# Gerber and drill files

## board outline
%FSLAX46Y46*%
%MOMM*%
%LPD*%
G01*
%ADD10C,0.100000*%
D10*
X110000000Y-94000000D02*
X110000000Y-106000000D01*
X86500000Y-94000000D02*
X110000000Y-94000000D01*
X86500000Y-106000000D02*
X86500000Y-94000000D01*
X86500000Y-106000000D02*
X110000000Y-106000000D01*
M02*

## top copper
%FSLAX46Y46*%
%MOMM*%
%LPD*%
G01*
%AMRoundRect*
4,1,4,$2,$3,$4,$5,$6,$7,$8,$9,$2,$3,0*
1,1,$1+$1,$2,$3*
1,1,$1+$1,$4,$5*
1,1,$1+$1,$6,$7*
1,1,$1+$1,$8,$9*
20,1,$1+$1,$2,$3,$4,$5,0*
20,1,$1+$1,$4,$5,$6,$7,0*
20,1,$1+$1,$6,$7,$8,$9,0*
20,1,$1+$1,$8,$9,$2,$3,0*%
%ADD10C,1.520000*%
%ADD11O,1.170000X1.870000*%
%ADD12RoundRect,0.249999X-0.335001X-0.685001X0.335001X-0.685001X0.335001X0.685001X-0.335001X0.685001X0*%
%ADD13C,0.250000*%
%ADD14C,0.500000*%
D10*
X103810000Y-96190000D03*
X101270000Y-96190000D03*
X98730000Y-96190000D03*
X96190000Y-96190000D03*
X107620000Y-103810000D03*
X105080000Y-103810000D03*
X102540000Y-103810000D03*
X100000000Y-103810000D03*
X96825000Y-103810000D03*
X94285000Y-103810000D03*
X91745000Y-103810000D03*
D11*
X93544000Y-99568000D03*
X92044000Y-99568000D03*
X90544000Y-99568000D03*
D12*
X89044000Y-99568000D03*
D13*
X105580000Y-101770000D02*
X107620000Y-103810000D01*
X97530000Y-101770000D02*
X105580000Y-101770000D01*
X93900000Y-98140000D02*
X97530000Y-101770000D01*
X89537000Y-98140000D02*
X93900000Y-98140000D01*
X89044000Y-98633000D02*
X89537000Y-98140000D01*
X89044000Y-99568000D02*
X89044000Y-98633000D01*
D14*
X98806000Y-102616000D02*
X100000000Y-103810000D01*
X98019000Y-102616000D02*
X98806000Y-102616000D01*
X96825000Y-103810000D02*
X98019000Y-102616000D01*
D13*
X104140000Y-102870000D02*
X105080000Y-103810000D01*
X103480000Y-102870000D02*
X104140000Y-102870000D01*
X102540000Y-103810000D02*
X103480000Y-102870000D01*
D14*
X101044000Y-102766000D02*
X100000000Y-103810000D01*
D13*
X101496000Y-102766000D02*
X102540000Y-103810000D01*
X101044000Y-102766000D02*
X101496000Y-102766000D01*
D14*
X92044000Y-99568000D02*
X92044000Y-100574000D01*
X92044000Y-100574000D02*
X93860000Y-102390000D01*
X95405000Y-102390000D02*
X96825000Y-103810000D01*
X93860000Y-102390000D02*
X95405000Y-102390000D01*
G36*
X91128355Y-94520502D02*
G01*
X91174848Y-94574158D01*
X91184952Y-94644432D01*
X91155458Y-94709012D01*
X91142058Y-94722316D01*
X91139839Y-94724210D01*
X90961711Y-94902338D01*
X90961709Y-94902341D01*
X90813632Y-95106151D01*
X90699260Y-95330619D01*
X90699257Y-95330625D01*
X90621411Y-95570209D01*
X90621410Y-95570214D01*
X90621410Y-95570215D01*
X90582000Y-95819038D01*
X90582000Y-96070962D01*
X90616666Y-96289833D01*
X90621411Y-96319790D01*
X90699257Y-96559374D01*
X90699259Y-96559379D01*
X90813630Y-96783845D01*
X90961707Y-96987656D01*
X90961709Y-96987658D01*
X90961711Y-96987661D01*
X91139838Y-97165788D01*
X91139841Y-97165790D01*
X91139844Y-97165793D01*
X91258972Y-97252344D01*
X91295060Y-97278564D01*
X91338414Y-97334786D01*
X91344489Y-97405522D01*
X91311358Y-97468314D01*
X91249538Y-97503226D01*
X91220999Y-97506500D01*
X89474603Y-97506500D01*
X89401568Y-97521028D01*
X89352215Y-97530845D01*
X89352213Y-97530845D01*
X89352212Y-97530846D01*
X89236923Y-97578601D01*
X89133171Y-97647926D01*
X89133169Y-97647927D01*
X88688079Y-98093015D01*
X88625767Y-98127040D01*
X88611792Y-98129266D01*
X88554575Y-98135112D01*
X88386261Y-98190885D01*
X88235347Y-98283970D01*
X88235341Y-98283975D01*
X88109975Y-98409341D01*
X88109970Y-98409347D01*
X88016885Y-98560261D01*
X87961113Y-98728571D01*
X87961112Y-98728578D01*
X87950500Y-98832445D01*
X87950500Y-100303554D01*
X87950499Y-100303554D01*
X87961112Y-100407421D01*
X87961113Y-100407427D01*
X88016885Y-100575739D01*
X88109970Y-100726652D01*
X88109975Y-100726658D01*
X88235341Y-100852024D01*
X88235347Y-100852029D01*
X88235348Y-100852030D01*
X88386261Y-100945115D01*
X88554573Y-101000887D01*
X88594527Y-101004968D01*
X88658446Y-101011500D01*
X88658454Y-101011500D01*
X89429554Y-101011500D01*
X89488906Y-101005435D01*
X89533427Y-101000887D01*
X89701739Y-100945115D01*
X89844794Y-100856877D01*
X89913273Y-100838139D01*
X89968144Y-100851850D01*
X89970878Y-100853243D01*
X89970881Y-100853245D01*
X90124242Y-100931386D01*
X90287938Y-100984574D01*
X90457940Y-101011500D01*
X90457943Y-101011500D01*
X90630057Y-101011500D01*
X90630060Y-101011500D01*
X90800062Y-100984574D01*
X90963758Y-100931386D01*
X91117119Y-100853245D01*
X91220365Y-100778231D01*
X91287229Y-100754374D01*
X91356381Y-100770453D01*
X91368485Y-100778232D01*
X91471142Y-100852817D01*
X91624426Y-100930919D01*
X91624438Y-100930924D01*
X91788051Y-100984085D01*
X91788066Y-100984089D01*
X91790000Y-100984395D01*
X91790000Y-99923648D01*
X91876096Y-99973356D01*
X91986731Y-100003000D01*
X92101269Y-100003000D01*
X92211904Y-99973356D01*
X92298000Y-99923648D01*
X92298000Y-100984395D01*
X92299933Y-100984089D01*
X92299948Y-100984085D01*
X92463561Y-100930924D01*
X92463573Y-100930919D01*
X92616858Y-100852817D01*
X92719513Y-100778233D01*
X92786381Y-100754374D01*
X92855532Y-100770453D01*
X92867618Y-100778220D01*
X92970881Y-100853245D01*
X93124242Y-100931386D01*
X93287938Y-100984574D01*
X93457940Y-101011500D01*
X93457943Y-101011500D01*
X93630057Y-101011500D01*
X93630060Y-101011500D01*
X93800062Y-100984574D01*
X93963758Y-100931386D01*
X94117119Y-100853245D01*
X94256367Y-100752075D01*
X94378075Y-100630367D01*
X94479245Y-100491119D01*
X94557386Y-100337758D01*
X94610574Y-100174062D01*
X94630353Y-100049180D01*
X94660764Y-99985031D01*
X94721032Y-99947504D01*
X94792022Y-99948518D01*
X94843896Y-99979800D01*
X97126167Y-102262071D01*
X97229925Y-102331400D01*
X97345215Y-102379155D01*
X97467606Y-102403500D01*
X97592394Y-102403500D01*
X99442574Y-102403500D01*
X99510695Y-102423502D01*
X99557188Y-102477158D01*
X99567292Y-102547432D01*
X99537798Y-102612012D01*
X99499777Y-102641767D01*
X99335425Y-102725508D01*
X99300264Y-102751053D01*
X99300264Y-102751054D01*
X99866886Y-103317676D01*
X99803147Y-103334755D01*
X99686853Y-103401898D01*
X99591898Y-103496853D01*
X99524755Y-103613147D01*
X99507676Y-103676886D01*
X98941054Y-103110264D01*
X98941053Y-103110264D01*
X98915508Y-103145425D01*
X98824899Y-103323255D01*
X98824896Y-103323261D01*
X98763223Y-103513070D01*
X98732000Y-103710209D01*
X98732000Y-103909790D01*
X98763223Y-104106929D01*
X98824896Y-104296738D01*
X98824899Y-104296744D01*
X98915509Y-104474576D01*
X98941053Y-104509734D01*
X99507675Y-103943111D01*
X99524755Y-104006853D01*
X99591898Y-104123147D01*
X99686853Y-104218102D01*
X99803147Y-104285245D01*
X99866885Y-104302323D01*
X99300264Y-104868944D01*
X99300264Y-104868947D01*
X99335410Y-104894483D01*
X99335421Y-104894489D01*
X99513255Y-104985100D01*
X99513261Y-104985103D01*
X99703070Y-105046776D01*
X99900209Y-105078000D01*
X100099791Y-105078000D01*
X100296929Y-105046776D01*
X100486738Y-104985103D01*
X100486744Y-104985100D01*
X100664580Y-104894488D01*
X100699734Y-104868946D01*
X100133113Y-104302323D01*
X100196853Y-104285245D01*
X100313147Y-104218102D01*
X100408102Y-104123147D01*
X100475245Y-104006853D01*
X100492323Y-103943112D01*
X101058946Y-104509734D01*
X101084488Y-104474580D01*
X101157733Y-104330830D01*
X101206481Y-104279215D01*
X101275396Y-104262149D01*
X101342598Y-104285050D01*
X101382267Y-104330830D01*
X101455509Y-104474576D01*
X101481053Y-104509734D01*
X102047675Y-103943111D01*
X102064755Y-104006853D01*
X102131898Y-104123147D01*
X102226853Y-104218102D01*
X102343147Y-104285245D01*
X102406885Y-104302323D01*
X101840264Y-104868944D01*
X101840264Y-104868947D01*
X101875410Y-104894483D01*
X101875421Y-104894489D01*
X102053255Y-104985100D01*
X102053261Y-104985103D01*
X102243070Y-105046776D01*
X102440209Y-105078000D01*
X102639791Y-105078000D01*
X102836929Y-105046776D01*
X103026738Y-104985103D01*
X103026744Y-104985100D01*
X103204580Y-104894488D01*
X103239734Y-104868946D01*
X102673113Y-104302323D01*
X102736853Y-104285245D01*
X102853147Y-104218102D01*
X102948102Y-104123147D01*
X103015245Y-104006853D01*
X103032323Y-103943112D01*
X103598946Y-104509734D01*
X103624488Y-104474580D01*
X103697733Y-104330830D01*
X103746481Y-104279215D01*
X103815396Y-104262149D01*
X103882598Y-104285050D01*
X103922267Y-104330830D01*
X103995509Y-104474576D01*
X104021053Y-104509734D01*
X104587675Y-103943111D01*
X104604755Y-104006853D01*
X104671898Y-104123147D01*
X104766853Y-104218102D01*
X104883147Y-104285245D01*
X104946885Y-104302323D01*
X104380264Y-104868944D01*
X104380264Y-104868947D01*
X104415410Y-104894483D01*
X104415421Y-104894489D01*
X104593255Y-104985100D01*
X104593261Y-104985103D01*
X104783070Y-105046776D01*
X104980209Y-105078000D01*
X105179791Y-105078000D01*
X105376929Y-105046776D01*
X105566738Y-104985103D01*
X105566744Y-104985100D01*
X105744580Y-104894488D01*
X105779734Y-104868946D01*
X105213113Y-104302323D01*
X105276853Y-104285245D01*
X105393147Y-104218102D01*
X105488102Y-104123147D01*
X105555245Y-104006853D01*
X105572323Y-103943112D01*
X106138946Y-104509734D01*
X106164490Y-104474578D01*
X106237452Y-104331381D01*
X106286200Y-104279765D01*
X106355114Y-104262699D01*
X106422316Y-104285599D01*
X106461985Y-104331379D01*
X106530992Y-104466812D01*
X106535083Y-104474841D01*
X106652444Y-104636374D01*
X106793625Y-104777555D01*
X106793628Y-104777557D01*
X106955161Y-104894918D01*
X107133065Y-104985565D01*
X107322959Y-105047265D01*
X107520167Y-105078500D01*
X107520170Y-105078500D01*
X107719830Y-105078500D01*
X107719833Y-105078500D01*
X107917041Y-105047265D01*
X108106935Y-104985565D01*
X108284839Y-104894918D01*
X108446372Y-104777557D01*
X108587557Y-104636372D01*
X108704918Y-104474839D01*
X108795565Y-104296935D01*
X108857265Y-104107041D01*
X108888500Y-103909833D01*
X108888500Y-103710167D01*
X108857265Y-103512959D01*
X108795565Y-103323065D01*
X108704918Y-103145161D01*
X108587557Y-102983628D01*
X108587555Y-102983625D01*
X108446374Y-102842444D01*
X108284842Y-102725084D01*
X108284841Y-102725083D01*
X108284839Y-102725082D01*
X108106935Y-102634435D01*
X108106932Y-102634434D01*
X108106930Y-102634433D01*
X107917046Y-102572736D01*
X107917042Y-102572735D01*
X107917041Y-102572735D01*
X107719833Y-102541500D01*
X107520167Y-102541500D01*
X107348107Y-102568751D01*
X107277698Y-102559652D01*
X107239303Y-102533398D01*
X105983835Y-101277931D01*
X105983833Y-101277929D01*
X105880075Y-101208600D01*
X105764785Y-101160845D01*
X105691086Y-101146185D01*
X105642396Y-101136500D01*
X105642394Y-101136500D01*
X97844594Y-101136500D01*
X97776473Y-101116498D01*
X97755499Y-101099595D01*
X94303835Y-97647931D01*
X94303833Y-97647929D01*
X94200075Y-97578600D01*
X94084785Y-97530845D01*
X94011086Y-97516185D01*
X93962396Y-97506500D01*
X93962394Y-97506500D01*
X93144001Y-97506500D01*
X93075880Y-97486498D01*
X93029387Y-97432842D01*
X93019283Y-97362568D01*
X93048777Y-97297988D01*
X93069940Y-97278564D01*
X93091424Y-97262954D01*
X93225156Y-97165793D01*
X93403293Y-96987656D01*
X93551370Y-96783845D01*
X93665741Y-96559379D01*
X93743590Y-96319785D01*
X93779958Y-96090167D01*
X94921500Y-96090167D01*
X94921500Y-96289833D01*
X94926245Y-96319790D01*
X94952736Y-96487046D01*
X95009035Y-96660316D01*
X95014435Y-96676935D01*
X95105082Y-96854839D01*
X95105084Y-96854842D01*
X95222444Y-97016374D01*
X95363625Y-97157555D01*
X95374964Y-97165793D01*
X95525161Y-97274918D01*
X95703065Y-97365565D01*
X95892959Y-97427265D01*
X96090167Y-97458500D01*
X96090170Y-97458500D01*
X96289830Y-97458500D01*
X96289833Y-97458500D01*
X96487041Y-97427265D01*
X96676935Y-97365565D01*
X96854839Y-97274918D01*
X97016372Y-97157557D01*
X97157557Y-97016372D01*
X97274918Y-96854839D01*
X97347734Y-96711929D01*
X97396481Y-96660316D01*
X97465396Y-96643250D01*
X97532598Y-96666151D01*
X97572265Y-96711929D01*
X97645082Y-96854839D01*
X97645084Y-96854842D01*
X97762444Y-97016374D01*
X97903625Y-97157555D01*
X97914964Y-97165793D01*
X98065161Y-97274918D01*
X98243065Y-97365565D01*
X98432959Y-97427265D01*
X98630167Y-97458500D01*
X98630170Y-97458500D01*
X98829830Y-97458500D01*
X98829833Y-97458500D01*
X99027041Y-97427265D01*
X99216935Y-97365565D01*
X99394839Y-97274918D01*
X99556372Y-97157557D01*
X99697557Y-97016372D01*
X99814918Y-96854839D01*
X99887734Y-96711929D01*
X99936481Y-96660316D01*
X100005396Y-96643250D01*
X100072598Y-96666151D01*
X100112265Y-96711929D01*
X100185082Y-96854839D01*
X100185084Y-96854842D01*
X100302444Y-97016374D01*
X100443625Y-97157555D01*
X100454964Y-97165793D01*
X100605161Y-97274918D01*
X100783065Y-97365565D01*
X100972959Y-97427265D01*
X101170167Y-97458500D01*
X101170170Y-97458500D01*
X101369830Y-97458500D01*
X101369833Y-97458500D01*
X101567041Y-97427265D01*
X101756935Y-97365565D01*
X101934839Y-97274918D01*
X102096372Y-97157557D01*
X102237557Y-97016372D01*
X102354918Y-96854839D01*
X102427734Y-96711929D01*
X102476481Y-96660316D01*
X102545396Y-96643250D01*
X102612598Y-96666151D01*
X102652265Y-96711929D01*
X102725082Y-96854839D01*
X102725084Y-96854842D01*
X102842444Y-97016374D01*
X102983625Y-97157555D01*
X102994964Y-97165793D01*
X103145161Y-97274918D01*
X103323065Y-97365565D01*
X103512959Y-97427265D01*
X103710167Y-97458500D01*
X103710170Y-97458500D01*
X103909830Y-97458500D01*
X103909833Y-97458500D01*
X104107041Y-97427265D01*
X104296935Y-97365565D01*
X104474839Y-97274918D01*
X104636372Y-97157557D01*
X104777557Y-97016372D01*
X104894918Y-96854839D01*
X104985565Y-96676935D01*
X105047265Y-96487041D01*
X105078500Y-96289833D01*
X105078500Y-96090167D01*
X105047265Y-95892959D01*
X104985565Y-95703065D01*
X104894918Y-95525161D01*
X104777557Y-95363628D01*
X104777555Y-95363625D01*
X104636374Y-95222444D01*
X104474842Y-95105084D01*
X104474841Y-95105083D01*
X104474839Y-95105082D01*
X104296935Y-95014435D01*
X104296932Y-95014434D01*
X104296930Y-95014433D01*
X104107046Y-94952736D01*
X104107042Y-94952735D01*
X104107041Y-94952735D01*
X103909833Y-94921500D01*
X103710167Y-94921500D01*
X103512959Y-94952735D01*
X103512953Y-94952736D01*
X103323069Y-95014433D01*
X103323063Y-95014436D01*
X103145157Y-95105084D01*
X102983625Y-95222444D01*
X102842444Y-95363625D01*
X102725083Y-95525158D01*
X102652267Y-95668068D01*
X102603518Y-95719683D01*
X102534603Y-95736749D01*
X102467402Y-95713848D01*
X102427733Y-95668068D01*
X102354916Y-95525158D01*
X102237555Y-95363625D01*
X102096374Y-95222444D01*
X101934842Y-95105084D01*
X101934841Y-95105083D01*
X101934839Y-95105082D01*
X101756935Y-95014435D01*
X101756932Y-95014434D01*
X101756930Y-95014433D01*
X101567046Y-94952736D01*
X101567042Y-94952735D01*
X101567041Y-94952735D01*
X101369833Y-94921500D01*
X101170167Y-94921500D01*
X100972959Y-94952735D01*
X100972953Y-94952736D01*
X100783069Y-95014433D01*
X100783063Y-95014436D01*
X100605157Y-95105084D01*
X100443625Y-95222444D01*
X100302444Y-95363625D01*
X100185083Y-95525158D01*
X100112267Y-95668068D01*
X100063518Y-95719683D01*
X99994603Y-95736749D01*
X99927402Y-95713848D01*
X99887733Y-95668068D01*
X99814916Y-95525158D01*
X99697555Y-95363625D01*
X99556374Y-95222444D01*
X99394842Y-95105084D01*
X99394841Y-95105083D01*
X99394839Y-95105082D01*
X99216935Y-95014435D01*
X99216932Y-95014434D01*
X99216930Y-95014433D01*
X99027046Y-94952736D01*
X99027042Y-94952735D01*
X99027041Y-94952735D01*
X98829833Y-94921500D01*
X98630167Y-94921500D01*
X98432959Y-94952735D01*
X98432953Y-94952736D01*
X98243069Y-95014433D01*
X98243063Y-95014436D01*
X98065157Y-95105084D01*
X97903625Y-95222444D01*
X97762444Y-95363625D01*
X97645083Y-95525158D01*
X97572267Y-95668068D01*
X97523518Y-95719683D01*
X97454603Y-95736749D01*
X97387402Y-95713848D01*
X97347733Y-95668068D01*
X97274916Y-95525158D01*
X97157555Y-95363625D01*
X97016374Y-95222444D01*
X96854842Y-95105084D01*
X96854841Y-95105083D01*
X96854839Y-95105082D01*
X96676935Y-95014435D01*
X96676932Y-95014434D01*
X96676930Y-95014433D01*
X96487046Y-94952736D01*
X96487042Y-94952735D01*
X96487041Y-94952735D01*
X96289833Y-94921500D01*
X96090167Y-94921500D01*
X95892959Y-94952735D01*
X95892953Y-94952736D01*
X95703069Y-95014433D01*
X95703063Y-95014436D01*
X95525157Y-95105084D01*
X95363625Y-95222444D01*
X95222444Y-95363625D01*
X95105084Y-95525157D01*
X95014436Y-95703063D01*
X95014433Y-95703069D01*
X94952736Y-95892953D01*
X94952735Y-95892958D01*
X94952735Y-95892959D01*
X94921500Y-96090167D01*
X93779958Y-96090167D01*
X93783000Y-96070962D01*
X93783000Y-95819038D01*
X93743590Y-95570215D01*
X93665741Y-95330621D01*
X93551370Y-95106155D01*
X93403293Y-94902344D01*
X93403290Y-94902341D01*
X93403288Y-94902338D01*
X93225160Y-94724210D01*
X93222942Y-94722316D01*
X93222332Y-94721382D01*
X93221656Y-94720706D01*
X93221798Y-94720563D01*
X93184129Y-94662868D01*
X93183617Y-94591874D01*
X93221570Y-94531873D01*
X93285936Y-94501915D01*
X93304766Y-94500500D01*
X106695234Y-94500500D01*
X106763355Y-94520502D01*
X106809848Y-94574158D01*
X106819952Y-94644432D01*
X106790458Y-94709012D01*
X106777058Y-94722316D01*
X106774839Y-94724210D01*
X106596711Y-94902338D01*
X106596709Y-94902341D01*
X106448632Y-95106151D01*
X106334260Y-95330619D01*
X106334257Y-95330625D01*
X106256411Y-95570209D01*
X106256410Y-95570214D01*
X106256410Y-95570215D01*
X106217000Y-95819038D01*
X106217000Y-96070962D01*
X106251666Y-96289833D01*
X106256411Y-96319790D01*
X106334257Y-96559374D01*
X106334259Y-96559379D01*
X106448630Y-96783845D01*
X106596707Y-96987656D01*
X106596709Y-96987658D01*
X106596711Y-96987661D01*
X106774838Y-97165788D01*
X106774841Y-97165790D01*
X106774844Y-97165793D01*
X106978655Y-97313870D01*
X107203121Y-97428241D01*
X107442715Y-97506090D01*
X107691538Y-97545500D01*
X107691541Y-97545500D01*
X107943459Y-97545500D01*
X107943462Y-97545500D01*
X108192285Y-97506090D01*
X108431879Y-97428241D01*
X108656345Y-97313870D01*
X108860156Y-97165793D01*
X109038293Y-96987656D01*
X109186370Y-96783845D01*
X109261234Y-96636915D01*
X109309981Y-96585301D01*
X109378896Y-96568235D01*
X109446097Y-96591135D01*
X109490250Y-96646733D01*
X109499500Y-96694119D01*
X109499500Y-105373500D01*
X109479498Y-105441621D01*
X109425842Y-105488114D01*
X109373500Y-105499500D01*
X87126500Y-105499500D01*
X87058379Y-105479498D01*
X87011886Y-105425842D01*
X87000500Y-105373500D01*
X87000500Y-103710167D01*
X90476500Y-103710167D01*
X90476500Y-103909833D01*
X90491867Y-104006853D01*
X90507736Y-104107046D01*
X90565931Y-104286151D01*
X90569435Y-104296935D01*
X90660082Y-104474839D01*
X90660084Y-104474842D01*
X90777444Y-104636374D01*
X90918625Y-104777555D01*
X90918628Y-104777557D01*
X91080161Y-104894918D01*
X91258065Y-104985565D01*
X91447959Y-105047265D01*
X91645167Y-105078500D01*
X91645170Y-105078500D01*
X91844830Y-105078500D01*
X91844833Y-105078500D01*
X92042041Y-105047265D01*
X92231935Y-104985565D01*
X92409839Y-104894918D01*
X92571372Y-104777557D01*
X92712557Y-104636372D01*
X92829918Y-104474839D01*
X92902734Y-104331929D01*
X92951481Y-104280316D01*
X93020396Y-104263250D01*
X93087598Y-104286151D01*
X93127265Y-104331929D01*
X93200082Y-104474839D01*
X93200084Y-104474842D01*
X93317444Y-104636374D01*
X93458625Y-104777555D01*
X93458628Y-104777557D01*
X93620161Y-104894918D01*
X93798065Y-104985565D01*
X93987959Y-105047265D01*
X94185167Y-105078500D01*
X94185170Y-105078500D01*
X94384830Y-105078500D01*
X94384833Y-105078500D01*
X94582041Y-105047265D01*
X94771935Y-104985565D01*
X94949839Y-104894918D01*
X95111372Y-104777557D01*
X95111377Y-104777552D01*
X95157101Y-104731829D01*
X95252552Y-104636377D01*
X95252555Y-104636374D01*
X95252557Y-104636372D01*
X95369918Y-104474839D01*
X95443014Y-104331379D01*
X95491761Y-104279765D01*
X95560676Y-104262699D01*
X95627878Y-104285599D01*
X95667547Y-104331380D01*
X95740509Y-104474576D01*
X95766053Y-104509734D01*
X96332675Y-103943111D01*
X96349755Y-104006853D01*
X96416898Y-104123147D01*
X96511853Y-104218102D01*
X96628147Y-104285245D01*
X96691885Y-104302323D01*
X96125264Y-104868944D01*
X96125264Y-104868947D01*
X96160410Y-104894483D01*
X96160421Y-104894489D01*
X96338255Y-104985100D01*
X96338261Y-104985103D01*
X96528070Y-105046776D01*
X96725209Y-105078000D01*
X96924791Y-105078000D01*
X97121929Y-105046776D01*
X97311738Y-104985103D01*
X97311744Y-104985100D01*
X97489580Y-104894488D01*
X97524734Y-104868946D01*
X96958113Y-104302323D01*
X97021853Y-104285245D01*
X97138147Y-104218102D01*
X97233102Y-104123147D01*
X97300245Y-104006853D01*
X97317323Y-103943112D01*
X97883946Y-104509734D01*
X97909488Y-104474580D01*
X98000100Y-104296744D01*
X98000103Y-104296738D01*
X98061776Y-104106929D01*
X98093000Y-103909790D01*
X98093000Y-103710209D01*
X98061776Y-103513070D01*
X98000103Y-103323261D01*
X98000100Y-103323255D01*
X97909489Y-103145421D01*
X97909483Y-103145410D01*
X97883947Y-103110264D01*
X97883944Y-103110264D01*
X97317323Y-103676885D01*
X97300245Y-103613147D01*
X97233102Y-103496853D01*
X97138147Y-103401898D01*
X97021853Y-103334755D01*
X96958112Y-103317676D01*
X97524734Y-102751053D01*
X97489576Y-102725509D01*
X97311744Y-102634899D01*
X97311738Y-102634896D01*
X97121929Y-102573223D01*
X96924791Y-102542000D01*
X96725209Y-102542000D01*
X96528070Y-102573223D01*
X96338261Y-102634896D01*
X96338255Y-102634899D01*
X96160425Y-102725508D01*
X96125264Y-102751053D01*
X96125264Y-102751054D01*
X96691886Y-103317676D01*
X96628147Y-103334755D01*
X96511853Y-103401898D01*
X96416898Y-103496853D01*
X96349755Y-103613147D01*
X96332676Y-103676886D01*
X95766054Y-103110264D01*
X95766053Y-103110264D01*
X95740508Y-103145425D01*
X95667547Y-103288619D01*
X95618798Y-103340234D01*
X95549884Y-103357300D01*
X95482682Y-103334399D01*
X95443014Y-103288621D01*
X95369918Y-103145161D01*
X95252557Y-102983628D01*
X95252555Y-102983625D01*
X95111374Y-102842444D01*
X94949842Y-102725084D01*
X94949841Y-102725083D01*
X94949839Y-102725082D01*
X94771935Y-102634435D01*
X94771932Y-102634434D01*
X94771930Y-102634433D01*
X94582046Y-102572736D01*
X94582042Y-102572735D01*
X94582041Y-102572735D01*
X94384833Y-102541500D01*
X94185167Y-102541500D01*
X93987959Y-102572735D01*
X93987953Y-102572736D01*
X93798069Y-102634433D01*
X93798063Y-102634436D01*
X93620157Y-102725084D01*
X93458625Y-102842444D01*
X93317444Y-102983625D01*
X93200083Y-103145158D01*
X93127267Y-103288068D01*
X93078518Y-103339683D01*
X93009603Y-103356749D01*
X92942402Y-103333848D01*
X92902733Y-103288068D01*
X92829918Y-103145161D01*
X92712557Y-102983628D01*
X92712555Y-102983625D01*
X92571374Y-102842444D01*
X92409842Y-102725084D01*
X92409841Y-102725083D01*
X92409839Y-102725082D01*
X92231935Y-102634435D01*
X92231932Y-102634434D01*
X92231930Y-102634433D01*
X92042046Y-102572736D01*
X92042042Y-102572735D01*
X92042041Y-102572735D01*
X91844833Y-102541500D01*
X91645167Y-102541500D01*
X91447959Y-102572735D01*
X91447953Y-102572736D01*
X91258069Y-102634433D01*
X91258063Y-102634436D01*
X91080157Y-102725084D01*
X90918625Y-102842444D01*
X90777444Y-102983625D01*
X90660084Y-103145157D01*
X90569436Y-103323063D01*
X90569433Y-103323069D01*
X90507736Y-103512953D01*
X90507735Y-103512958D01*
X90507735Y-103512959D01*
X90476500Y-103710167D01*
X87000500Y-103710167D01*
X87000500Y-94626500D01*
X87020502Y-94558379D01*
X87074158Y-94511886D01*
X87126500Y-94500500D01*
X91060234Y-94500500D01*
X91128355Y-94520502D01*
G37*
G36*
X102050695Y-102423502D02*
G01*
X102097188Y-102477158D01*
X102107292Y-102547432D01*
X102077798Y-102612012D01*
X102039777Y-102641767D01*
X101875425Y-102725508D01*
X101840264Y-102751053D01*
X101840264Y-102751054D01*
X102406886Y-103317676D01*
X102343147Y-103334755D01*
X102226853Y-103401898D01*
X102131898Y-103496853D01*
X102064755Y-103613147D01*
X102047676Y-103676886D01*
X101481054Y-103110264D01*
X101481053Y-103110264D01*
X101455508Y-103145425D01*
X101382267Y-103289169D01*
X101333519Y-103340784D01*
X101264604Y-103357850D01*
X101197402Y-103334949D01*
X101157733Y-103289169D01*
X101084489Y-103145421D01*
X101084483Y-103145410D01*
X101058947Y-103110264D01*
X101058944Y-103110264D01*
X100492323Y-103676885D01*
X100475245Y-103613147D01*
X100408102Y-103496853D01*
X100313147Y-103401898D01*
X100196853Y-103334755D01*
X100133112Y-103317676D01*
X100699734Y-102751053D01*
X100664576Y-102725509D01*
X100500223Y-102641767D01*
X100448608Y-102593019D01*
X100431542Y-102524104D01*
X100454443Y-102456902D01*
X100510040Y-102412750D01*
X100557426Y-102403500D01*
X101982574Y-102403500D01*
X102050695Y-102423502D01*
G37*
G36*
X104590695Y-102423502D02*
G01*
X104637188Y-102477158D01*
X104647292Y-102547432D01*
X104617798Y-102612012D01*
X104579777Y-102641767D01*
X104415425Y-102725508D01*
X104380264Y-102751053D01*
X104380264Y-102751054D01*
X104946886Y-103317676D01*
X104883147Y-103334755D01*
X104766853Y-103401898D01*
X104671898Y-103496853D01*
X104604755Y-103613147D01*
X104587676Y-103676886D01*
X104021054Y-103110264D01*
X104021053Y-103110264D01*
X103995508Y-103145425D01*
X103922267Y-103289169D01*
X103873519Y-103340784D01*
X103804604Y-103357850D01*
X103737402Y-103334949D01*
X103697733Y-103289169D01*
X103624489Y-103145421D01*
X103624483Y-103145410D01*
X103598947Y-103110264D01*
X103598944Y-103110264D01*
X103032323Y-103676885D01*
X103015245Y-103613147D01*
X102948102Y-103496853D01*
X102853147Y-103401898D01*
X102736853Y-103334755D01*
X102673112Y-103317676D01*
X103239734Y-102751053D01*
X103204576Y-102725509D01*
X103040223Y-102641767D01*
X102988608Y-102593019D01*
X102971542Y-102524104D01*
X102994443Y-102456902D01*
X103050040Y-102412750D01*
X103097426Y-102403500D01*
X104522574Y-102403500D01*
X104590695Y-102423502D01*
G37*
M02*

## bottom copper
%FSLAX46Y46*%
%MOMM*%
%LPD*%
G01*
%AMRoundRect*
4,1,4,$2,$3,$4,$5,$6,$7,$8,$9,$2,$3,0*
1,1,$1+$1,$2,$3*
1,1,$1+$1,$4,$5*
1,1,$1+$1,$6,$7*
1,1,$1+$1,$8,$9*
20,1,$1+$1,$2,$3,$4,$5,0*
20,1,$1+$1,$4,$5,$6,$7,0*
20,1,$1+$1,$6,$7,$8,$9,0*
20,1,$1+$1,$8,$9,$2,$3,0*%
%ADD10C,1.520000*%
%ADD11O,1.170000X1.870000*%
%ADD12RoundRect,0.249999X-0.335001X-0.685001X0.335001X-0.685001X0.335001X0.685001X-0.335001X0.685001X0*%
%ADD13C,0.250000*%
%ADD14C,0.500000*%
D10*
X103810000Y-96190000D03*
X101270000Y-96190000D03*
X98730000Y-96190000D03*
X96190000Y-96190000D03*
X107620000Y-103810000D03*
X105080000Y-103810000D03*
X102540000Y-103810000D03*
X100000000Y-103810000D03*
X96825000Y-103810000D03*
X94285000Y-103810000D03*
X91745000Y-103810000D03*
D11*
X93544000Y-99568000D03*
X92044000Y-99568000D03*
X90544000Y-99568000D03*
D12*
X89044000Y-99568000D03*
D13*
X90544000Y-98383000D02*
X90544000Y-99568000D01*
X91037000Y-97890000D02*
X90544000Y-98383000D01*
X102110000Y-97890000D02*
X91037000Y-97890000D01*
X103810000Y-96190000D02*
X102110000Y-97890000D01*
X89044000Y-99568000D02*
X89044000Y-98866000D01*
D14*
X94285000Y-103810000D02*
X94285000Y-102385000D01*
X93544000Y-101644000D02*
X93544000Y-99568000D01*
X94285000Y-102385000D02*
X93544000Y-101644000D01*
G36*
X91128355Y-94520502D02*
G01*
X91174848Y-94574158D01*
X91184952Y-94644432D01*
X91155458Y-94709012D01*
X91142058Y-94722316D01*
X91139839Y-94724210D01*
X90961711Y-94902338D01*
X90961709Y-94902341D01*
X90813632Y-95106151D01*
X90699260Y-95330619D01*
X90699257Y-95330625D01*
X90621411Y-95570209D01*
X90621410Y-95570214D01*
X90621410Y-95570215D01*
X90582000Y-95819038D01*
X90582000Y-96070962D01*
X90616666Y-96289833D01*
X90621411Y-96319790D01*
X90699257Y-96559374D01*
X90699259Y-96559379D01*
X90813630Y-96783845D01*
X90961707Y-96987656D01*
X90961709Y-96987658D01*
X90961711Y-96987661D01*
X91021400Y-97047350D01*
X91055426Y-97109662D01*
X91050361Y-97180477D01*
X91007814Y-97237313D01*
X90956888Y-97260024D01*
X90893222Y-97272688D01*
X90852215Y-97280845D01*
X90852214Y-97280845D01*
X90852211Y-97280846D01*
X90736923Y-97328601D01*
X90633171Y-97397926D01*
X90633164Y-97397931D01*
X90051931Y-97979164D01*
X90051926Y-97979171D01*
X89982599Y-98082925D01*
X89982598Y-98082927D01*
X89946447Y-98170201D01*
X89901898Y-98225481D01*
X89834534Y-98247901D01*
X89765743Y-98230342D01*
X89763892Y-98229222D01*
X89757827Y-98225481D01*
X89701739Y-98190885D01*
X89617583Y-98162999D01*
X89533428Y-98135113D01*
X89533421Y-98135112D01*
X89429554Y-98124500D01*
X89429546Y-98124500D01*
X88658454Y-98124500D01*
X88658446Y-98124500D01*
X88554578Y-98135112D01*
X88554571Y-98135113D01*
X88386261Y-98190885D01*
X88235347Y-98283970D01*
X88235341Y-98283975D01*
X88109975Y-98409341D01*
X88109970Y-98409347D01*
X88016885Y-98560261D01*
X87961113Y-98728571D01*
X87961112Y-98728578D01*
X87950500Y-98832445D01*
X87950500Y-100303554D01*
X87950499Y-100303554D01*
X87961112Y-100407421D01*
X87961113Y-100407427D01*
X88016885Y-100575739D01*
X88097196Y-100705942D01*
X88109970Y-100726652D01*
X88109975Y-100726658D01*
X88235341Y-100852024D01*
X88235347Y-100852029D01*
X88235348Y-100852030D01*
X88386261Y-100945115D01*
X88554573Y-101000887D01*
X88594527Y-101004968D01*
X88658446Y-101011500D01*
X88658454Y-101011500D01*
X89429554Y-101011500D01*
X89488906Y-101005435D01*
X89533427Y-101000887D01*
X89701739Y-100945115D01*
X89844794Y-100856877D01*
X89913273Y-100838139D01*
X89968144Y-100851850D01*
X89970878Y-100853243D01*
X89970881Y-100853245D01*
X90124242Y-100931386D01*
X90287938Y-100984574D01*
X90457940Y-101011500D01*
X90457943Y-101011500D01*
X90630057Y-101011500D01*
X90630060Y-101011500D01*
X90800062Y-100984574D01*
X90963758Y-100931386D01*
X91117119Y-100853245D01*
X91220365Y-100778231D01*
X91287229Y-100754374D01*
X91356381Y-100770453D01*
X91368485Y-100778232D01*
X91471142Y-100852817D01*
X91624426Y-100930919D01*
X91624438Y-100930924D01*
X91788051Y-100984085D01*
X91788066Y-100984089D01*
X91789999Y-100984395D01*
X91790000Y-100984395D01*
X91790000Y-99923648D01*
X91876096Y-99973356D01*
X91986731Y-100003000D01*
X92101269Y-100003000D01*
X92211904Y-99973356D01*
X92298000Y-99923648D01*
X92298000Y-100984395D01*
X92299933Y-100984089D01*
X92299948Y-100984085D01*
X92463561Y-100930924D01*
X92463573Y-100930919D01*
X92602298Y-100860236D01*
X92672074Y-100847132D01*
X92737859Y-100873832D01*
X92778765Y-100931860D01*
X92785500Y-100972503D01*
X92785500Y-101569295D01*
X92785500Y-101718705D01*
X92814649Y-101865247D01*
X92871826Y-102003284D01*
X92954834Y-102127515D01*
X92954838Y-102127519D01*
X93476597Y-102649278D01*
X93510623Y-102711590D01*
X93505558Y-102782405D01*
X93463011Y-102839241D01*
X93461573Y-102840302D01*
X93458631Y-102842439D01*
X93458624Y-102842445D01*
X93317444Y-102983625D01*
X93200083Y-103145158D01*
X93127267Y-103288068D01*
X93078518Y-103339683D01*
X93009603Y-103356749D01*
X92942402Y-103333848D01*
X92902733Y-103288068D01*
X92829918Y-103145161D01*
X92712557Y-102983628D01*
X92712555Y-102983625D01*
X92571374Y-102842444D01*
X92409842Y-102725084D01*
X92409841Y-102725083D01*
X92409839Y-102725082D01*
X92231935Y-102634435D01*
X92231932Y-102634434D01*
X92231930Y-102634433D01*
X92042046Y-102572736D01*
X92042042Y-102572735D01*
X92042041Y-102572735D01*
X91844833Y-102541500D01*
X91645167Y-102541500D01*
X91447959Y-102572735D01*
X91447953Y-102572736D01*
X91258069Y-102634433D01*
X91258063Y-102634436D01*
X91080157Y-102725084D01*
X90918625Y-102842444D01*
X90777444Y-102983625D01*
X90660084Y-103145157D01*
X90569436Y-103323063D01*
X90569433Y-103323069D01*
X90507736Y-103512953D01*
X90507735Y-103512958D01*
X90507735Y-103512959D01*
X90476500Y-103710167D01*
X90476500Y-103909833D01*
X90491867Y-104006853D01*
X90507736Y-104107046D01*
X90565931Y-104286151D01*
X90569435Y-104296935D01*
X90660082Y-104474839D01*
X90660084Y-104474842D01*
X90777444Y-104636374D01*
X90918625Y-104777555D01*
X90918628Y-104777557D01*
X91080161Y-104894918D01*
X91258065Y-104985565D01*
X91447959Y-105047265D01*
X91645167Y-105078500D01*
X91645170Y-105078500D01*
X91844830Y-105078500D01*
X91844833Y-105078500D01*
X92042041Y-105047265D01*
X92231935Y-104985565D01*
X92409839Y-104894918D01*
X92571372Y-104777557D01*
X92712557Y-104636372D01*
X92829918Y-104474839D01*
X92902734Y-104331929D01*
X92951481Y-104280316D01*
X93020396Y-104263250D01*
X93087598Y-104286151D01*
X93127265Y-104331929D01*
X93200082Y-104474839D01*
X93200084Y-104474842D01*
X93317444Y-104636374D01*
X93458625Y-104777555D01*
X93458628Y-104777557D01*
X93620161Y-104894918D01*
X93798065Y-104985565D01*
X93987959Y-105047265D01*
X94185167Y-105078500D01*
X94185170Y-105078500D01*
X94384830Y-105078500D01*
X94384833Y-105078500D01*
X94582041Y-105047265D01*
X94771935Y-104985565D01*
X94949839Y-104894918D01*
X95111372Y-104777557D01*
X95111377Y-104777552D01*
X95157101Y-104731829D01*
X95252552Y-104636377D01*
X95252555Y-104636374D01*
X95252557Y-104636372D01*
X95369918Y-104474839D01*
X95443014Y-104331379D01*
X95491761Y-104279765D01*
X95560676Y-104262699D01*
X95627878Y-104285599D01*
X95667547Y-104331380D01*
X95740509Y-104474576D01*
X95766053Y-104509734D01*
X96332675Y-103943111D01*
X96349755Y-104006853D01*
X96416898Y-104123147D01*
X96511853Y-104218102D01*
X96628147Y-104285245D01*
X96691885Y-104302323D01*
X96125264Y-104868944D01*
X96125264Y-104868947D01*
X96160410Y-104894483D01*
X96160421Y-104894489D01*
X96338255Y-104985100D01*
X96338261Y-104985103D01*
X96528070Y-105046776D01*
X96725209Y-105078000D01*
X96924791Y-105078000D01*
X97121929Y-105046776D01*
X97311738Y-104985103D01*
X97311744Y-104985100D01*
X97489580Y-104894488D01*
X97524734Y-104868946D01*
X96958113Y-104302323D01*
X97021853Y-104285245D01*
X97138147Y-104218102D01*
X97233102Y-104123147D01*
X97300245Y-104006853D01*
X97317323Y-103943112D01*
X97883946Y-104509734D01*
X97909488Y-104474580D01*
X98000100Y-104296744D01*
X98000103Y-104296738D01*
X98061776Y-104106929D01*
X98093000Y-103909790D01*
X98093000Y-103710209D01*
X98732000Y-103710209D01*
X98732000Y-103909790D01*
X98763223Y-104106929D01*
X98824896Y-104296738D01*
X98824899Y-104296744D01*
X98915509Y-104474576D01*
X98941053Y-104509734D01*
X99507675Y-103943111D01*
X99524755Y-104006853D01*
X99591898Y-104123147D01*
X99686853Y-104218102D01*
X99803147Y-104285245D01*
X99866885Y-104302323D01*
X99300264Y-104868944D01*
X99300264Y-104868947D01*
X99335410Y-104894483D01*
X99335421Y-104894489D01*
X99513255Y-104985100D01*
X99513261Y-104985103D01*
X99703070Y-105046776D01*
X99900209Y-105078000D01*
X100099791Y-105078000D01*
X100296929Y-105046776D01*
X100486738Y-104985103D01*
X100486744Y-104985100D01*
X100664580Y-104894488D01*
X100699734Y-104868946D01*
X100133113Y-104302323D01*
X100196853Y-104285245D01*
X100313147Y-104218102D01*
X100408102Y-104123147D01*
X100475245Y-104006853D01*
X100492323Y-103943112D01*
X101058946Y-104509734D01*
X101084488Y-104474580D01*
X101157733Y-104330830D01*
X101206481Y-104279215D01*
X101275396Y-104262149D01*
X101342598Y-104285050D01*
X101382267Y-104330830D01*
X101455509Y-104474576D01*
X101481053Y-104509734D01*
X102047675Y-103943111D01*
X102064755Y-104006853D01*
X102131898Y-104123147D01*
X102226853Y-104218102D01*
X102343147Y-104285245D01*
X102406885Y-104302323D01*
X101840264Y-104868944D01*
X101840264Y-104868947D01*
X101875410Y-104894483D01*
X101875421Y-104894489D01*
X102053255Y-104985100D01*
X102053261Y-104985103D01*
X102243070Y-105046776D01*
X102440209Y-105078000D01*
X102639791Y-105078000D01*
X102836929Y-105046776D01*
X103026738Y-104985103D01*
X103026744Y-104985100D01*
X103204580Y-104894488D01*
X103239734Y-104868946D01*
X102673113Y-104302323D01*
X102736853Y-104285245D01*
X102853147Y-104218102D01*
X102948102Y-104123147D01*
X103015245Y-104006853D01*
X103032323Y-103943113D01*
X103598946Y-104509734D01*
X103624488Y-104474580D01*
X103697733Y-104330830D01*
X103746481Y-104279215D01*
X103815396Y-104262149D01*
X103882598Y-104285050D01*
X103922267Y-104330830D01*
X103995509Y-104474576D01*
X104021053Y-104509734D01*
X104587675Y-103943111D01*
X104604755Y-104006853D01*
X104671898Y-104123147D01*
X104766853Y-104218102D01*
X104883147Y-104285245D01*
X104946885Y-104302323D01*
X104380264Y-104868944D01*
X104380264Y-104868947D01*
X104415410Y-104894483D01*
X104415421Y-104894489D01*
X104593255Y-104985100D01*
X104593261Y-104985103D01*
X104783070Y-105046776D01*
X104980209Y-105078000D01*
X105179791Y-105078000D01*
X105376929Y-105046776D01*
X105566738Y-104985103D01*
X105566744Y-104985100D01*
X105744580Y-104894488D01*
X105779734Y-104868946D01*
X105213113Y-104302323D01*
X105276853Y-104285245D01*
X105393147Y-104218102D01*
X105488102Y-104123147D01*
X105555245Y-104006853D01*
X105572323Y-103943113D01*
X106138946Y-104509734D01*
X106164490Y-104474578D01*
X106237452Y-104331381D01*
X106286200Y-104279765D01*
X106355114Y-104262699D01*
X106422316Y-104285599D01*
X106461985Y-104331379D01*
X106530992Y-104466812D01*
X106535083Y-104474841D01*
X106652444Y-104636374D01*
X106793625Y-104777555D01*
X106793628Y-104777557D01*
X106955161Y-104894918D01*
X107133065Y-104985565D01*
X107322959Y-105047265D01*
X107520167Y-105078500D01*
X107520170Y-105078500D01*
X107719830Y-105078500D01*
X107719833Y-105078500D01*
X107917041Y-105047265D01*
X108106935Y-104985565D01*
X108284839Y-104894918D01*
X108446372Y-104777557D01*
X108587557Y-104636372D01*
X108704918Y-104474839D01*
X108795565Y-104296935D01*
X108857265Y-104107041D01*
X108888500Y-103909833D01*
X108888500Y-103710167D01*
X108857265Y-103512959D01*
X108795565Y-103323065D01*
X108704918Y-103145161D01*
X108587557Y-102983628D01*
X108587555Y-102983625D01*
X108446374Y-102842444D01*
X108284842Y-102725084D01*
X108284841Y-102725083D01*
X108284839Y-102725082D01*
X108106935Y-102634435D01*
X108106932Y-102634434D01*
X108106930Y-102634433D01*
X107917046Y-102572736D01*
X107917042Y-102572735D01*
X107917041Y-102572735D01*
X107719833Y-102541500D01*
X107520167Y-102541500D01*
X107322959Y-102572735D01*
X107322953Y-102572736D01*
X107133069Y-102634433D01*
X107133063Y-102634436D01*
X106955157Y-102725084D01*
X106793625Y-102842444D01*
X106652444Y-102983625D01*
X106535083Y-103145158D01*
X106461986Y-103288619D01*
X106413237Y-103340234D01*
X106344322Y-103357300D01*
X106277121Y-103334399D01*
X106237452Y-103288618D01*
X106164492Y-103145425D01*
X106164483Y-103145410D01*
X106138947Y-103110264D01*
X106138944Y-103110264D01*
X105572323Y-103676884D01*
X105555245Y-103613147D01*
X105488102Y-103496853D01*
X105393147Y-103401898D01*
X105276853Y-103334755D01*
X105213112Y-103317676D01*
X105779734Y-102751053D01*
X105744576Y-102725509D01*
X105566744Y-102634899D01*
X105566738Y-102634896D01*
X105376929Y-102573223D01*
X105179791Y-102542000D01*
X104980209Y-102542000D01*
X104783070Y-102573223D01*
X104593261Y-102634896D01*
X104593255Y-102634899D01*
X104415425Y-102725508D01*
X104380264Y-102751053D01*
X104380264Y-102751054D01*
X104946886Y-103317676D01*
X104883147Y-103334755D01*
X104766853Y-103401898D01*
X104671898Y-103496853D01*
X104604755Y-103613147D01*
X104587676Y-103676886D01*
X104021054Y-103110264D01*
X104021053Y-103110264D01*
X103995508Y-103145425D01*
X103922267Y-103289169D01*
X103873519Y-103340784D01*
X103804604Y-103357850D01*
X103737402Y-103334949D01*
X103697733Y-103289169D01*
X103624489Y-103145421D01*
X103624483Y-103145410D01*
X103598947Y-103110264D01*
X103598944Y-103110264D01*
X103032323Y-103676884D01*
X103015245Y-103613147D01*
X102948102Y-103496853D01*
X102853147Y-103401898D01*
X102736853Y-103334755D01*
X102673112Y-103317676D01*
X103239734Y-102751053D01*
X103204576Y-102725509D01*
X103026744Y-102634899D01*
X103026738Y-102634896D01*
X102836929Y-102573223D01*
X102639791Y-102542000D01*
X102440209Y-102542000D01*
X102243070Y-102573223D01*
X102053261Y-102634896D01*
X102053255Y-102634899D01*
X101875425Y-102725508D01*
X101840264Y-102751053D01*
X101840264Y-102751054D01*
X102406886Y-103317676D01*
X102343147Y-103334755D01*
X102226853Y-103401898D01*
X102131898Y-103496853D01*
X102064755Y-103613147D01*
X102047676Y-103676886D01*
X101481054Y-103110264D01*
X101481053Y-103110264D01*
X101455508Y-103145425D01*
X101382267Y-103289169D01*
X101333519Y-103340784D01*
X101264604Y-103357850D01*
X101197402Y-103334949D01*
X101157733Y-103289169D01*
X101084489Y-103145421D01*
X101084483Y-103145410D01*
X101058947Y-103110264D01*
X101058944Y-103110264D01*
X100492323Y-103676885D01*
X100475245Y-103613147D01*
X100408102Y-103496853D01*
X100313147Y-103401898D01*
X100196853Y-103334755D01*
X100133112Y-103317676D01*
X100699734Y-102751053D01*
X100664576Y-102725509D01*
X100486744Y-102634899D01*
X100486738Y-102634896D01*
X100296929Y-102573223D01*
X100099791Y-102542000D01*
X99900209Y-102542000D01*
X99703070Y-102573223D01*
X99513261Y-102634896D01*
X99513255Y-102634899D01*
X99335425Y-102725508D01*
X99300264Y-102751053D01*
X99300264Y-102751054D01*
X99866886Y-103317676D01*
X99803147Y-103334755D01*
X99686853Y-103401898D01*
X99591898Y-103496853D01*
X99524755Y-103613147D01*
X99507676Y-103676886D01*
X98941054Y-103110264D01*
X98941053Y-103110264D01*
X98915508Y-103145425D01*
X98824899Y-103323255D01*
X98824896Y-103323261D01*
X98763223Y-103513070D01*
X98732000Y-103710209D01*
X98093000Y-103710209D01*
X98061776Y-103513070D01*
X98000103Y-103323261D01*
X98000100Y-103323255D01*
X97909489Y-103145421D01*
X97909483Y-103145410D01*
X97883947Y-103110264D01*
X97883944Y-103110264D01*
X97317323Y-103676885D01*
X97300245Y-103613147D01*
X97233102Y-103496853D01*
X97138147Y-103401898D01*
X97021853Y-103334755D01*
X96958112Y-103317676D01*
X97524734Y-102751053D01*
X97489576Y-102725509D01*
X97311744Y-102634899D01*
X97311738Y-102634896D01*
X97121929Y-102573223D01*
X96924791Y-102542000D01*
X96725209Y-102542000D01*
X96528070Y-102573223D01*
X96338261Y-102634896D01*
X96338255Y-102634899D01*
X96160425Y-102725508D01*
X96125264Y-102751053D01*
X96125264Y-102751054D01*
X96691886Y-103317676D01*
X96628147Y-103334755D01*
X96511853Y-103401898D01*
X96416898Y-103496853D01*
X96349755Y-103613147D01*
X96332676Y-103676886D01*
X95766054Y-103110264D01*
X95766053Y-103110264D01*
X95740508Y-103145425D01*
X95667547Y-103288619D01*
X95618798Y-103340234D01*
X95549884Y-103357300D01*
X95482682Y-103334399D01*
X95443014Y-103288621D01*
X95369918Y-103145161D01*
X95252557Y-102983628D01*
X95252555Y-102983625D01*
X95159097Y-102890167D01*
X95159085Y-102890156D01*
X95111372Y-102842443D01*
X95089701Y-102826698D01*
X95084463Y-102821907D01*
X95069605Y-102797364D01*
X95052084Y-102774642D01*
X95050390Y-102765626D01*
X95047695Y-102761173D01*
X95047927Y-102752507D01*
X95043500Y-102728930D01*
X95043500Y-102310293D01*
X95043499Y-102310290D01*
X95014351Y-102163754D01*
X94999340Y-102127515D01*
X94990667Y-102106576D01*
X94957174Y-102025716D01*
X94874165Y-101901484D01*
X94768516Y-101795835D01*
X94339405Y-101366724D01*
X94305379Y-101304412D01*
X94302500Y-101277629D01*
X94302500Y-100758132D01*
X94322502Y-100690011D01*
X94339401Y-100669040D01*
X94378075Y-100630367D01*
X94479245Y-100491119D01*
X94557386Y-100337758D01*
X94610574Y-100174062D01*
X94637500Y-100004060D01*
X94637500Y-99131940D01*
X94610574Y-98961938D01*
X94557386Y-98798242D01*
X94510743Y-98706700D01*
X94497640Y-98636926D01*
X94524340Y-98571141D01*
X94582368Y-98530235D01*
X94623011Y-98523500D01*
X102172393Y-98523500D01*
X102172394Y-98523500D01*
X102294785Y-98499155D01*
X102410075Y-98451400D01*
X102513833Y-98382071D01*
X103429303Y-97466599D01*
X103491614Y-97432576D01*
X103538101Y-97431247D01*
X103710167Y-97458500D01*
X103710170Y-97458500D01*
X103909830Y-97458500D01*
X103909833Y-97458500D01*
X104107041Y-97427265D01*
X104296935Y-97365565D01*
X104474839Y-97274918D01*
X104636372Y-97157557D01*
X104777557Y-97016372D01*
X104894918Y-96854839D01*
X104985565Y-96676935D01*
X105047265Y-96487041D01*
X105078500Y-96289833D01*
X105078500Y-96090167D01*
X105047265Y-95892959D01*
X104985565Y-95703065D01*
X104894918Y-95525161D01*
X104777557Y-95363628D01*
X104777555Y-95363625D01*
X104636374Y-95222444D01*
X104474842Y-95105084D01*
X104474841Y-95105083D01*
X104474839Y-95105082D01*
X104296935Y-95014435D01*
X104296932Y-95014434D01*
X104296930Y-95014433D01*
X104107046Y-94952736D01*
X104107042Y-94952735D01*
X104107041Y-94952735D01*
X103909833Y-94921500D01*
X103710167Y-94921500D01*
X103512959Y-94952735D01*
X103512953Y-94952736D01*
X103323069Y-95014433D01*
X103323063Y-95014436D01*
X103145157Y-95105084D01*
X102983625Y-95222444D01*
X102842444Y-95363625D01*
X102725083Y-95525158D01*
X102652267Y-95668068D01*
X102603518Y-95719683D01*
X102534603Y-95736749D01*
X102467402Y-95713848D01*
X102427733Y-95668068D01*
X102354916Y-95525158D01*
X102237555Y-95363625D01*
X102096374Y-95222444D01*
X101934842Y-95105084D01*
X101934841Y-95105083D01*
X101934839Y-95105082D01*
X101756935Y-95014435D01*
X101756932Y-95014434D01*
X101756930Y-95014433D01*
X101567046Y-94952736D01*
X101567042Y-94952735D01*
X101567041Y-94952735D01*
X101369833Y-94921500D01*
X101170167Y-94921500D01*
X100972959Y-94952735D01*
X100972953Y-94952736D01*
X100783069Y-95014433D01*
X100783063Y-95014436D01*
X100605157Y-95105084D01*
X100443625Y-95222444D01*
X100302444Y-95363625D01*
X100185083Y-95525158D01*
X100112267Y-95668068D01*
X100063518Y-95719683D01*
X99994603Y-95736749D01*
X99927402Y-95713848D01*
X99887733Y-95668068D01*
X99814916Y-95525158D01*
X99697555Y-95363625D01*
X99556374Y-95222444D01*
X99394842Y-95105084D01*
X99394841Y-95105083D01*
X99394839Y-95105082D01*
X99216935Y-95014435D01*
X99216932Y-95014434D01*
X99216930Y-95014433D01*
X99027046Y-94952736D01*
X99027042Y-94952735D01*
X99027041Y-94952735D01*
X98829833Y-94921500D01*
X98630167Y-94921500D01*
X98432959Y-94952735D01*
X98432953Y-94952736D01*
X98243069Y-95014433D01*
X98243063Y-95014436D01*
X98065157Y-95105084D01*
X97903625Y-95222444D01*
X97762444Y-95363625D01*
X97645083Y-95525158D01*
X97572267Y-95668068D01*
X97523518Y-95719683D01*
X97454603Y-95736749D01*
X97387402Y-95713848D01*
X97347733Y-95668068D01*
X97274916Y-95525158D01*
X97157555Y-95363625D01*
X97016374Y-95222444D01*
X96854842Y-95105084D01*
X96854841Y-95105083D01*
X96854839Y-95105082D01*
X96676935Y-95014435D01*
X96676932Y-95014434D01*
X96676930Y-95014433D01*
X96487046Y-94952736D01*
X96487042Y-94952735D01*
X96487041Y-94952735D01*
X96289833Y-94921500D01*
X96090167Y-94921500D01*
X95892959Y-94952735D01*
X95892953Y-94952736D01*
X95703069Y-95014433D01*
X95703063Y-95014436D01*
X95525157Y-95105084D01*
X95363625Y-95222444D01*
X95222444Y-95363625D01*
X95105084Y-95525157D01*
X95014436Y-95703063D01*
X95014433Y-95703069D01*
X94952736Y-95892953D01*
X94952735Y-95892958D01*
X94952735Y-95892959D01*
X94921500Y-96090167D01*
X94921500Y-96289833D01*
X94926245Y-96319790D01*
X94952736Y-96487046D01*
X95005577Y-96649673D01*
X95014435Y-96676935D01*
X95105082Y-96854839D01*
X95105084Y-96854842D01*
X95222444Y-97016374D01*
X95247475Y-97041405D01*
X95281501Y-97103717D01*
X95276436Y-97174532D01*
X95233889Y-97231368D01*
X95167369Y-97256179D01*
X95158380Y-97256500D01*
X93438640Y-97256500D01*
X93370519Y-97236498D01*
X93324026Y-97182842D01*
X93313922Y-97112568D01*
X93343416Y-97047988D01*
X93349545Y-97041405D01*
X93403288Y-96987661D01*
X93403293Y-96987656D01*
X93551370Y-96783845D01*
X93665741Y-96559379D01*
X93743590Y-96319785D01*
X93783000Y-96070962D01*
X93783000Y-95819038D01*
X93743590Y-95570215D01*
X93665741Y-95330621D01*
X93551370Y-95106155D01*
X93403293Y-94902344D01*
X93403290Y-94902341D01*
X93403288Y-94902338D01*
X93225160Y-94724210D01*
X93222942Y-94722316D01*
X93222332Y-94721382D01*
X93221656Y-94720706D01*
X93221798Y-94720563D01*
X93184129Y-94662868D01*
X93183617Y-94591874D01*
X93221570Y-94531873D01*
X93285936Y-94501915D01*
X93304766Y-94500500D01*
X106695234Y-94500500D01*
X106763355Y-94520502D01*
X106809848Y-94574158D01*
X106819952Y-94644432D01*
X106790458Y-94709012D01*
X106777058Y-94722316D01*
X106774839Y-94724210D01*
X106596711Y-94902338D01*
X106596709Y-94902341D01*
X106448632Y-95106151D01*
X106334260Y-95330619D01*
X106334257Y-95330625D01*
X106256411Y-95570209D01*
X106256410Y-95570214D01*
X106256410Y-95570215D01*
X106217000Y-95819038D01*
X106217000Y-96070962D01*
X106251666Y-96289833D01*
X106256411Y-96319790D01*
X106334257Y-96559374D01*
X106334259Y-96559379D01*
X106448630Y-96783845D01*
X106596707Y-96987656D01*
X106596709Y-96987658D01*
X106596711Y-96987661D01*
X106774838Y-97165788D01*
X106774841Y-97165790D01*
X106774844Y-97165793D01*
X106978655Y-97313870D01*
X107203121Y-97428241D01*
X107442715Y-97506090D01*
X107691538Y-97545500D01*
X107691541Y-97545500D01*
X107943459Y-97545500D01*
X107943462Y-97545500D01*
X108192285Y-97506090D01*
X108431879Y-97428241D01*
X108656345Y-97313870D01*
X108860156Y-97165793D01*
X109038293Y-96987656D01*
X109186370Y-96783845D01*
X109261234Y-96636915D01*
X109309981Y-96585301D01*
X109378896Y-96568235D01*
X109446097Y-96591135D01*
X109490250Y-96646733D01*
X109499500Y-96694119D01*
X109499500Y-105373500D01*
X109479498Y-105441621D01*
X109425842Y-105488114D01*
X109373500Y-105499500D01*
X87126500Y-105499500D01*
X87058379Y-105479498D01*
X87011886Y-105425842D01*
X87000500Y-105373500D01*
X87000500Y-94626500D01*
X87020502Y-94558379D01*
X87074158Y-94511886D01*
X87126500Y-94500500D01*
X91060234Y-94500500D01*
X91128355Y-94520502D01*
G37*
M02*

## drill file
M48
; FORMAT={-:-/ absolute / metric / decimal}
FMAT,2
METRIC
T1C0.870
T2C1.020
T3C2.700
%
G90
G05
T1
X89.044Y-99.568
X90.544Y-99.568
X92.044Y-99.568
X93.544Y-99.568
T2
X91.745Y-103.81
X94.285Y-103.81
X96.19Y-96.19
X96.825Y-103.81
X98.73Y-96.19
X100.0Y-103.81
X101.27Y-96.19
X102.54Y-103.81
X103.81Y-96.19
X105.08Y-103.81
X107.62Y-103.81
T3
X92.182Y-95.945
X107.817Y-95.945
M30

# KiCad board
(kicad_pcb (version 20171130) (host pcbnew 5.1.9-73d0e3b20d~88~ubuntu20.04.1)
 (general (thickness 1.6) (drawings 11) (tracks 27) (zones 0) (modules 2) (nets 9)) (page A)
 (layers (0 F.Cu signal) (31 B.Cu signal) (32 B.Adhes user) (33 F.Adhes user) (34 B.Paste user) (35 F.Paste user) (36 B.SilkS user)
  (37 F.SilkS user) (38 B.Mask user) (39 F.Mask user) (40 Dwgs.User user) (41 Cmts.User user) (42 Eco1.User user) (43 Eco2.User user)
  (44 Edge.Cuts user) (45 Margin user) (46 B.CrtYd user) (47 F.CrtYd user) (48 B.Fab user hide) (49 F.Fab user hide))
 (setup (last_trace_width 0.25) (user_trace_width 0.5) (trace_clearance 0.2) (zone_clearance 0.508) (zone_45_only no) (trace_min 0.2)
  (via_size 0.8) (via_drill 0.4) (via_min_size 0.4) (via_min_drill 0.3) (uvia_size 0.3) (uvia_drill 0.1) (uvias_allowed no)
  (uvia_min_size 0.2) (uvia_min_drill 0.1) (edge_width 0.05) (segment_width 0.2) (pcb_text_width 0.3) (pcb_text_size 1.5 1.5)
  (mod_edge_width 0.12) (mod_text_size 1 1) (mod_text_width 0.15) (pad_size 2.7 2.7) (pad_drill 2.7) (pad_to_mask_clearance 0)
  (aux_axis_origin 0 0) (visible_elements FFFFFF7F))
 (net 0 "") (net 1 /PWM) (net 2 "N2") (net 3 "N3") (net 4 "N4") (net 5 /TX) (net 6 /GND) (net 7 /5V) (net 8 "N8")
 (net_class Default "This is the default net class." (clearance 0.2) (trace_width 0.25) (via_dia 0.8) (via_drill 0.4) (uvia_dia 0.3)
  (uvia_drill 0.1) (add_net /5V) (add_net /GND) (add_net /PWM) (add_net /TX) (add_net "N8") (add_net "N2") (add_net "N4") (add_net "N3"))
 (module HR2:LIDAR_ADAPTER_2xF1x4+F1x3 (layer F.Cu) (at 100 100)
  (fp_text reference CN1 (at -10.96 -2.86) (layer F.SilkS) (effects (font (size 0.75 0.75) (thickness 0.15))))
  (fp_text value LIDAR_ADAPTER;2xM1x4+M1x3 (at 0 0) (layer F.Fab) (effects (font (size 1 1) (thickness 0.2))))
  (pad "" np_thru_hole circle (at -7.8175 -4.055) (size 2.7 2.7) (drill 2.7) (layers *.Cu *.Mask))
  (pad "" np_thru_hole circle (at 7.8175 -4.055) (size 2.7 2.7) (drill 2.7) (layers *.Cu *.Mask))
  (pad 11 thru_hole circle (at 3.81 -3.81) (size 1.52 1.52) (drill 1.02) (layers *.Cu *.Mask) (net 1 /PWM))
  (pad 10 thru_hole circle (at 1.27 -3.81) (size 1.52 1.52) (drill 1.02) (layers *.Cu *.Mask) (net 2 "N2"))
  (pad 9 thru_hole circle (at -1.27 -3.81) (size 1.52 1.52) (drill 1.02) (layers *.Cu *.Mask) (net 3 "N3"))
  (pad 8 thru_hole circle (at -3.81 -3.81) (size 1.52 1.52) (drill 1.02) (layers *.Cu *.Mask) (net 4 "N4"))
  (pad 7 thru_hole circle (at 7.62 3.81) (size 1.52 1.52) (drill 1.02) (layers *.Cu *.Mask) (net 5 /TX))
  (pad 6 thru_hole circle (at 5.08 3.81) (size 1.52 1.52) (drill 1.02) (layers *.Cu *.Mask) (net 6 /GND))
  (pad 5 thru_hole circle (at 2.54 3.81) (size 1.52 1.52) (drill 1.02) (layers *.Cu *.Mask) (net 6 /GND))
  (pad 4 thru_hole circle (at 0 3.81) (size 1.52 1.52) (drill 1.02) (layers *.Cu *.Mask) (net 6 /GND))
  (pad 3 thru_hole circle (at -3.175 3.81) (size 1.52 1.52) (drill 1.02) (layers *.Cu *.Mask) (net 6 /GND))
  (pad 2 thru_hole circle (at -5.715 3.81) (size 1.52 1.52) (drill 1.02) (layers *.Cu *.Mask) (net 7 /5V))
  (pad 1 thru_hole circle (at -8.255 3.81) (size 1.52 1.52) (drill 1.02) (layers *.Cu *.Mask) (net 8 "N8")))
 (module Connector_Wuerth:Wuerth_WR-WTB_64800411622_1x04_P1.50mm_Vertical (layer F.Cu) (at 89.044 99.568)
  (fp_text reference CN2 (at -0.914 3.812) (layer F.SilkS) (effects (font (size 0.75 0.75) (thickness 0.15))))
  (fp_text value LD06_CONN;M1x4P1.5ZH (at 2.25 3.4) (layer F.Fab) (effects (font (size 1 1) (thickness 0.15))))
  (pad 4 thru_hole oval (at 4.5 0) (size 1.17 1.87) (drill 0.87) (layers *.Cu *.Mask) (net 7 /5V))
  (pad 3 thru_hole oval (at 3 0) (size 1.17 1.87) (drill 0.87) (layers *.Cu *.Mask) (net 6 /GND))
  (pad 2 thru_hole oval (at 1.5 0) (size 1.17 1.87) (drill 0.87) (layers *.Cu *.Mask) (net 1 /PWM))
  (pad 1 thru_hole roundrect (at 0 0) (size 1.17 1.87) (drill 0.87) (layers *.Cu *.Mask) (roundrect_rratio 0.213674358974359) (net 5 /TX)))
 (gr_line (start 110 94) (end 110 106) (layer Edge.Cuts) (width 0.1))
 (gr_line (start 86.5 94) (end 110 94) (layer Edge.Cuts) (width 0.1))
 (gr_line (start 86.5 106) (end 86.5 94) (layer Edge.Cuts) (width 0.1))
 (gr_line (start 86.5 106) (end 110 106) (layer Edge.Cuts) (width 0.1))
 (segment (start 90.544 98.383) (end 90.544 99.568) (width 0.25) (layer B.Cu) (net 1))
 (segment (start 91.037 97.89) (end 90.544 98.383) (width 0.25) (layer B.Cu) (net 1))
 (segment (start 102.11 97.89) (end 91.037 97.89) (width 0.25) (layer B.Cu) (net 1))
 (segment (start 103.81 96.19) (end 102.11 97.89) (width 0.25) (layer B.Cu) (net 1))
 (segment (start 89.044 99.568) (end 89.044 98.866) (width 0.25) (layer B.Cu) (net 5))
 (segment (start 105.58 101.77) (end 107.62 103.81) (width 0.25) (layer F.Cu) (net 5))
 (segment (start 97.53 101.77) (end 105.58 101.77) (width 0.25) (layer F.Cu) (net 5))
 (segment (start 93.9 98.14) (end 97.53 101.77) (width 0.25) (layer F.Cu) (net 5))
 (segment (start 89.537 98.14) (end 93.9 98.14) (width 0.25) (layer F.Cu) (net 5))
 (segment (start 89.044 98.633) (end 89.537 98.14) (width 0.25) (layer F.Cu) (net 5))
 (segment (start 89.044 99.568) (end 89.044 98.633) (width 0.25) (layer F.Cu) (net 5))
 (segment (start 98.806 102.616) (end 100 103.81) (width 0.5) (layer F.Cu) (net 6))
 (segment (start 98.019 102.616) (end 98.806 102.616) (width 0.5) (layer F.Cu) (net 6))
 (segment (start 96.825 103.81) (end 98.019 102.616) (width 0.5) (layer F.Cu) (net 6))
 (segment (start 104.14 102.87) (end 105.08 103.81) (width 0.25) (layer F.Cu) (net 6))
 (segment (start 103.48 102.87) (end 104.14 102.87) (width 0.25) (layer F.Cu) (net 6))
 (segment (start 102.54 103.81) (end 103.48 102.87) (width 0.25) (layer F.Cu) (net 6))
 (segment (start 101.044 102.766) (end 100 103.81) (width 0.5) (layer F.Cu) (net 6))
 (segment (start 101.496 102.766) (end 102.54 103.81) (width 0.25) (layer F.Cu) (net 6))
 (segment (start 101.044 102.766) (end 101.496 102.766) (width 0.25) (layer F.Cu) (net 6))
 (segment (start 92.044 99.568) (end 92.044 100.574) (width 0.5) (layer F.Cu) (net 6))
 (segment (start 92.044 100.574) (end 93.86 102.39) (width 0.5) (layer F.Cu) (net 6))
 (segment (start 95.405 102.39) (end 96.825 103.81) (width 0.5) (layer F.Cu) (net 6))
 (segment (start 93.86 102.39) (end 95.405 102.39) (width 0.5) (layer F.Cu) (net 6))
 (segment (start 94.285 103.81) (end 94.285 102.385) (width 0.5) (layer B.Cu) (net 7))
 (segment (start 93.544 101.644) (end 93.544 99.568) (width 0.5) (layer B.Cu) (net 7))
 (segment (start 94.285 102.385) (end 93.544 101.644) (width 0.5) (layer B.Cu) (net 7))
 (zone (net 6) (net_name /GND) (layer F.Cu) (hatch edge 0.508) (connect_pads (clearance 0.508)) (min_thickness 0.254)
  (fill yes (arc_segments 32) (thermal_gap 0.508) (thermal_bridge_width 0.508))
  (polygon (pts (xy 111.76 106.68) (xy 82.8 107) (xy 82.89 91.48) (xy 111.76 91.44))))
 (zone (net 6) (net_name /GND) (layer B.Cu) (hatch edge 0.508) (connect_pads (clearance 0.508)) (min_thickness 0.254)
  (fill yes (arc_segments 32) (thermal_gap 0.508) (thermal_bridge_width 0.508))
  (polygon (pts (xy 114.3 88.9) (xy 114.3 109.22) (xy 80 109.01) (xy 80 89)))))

